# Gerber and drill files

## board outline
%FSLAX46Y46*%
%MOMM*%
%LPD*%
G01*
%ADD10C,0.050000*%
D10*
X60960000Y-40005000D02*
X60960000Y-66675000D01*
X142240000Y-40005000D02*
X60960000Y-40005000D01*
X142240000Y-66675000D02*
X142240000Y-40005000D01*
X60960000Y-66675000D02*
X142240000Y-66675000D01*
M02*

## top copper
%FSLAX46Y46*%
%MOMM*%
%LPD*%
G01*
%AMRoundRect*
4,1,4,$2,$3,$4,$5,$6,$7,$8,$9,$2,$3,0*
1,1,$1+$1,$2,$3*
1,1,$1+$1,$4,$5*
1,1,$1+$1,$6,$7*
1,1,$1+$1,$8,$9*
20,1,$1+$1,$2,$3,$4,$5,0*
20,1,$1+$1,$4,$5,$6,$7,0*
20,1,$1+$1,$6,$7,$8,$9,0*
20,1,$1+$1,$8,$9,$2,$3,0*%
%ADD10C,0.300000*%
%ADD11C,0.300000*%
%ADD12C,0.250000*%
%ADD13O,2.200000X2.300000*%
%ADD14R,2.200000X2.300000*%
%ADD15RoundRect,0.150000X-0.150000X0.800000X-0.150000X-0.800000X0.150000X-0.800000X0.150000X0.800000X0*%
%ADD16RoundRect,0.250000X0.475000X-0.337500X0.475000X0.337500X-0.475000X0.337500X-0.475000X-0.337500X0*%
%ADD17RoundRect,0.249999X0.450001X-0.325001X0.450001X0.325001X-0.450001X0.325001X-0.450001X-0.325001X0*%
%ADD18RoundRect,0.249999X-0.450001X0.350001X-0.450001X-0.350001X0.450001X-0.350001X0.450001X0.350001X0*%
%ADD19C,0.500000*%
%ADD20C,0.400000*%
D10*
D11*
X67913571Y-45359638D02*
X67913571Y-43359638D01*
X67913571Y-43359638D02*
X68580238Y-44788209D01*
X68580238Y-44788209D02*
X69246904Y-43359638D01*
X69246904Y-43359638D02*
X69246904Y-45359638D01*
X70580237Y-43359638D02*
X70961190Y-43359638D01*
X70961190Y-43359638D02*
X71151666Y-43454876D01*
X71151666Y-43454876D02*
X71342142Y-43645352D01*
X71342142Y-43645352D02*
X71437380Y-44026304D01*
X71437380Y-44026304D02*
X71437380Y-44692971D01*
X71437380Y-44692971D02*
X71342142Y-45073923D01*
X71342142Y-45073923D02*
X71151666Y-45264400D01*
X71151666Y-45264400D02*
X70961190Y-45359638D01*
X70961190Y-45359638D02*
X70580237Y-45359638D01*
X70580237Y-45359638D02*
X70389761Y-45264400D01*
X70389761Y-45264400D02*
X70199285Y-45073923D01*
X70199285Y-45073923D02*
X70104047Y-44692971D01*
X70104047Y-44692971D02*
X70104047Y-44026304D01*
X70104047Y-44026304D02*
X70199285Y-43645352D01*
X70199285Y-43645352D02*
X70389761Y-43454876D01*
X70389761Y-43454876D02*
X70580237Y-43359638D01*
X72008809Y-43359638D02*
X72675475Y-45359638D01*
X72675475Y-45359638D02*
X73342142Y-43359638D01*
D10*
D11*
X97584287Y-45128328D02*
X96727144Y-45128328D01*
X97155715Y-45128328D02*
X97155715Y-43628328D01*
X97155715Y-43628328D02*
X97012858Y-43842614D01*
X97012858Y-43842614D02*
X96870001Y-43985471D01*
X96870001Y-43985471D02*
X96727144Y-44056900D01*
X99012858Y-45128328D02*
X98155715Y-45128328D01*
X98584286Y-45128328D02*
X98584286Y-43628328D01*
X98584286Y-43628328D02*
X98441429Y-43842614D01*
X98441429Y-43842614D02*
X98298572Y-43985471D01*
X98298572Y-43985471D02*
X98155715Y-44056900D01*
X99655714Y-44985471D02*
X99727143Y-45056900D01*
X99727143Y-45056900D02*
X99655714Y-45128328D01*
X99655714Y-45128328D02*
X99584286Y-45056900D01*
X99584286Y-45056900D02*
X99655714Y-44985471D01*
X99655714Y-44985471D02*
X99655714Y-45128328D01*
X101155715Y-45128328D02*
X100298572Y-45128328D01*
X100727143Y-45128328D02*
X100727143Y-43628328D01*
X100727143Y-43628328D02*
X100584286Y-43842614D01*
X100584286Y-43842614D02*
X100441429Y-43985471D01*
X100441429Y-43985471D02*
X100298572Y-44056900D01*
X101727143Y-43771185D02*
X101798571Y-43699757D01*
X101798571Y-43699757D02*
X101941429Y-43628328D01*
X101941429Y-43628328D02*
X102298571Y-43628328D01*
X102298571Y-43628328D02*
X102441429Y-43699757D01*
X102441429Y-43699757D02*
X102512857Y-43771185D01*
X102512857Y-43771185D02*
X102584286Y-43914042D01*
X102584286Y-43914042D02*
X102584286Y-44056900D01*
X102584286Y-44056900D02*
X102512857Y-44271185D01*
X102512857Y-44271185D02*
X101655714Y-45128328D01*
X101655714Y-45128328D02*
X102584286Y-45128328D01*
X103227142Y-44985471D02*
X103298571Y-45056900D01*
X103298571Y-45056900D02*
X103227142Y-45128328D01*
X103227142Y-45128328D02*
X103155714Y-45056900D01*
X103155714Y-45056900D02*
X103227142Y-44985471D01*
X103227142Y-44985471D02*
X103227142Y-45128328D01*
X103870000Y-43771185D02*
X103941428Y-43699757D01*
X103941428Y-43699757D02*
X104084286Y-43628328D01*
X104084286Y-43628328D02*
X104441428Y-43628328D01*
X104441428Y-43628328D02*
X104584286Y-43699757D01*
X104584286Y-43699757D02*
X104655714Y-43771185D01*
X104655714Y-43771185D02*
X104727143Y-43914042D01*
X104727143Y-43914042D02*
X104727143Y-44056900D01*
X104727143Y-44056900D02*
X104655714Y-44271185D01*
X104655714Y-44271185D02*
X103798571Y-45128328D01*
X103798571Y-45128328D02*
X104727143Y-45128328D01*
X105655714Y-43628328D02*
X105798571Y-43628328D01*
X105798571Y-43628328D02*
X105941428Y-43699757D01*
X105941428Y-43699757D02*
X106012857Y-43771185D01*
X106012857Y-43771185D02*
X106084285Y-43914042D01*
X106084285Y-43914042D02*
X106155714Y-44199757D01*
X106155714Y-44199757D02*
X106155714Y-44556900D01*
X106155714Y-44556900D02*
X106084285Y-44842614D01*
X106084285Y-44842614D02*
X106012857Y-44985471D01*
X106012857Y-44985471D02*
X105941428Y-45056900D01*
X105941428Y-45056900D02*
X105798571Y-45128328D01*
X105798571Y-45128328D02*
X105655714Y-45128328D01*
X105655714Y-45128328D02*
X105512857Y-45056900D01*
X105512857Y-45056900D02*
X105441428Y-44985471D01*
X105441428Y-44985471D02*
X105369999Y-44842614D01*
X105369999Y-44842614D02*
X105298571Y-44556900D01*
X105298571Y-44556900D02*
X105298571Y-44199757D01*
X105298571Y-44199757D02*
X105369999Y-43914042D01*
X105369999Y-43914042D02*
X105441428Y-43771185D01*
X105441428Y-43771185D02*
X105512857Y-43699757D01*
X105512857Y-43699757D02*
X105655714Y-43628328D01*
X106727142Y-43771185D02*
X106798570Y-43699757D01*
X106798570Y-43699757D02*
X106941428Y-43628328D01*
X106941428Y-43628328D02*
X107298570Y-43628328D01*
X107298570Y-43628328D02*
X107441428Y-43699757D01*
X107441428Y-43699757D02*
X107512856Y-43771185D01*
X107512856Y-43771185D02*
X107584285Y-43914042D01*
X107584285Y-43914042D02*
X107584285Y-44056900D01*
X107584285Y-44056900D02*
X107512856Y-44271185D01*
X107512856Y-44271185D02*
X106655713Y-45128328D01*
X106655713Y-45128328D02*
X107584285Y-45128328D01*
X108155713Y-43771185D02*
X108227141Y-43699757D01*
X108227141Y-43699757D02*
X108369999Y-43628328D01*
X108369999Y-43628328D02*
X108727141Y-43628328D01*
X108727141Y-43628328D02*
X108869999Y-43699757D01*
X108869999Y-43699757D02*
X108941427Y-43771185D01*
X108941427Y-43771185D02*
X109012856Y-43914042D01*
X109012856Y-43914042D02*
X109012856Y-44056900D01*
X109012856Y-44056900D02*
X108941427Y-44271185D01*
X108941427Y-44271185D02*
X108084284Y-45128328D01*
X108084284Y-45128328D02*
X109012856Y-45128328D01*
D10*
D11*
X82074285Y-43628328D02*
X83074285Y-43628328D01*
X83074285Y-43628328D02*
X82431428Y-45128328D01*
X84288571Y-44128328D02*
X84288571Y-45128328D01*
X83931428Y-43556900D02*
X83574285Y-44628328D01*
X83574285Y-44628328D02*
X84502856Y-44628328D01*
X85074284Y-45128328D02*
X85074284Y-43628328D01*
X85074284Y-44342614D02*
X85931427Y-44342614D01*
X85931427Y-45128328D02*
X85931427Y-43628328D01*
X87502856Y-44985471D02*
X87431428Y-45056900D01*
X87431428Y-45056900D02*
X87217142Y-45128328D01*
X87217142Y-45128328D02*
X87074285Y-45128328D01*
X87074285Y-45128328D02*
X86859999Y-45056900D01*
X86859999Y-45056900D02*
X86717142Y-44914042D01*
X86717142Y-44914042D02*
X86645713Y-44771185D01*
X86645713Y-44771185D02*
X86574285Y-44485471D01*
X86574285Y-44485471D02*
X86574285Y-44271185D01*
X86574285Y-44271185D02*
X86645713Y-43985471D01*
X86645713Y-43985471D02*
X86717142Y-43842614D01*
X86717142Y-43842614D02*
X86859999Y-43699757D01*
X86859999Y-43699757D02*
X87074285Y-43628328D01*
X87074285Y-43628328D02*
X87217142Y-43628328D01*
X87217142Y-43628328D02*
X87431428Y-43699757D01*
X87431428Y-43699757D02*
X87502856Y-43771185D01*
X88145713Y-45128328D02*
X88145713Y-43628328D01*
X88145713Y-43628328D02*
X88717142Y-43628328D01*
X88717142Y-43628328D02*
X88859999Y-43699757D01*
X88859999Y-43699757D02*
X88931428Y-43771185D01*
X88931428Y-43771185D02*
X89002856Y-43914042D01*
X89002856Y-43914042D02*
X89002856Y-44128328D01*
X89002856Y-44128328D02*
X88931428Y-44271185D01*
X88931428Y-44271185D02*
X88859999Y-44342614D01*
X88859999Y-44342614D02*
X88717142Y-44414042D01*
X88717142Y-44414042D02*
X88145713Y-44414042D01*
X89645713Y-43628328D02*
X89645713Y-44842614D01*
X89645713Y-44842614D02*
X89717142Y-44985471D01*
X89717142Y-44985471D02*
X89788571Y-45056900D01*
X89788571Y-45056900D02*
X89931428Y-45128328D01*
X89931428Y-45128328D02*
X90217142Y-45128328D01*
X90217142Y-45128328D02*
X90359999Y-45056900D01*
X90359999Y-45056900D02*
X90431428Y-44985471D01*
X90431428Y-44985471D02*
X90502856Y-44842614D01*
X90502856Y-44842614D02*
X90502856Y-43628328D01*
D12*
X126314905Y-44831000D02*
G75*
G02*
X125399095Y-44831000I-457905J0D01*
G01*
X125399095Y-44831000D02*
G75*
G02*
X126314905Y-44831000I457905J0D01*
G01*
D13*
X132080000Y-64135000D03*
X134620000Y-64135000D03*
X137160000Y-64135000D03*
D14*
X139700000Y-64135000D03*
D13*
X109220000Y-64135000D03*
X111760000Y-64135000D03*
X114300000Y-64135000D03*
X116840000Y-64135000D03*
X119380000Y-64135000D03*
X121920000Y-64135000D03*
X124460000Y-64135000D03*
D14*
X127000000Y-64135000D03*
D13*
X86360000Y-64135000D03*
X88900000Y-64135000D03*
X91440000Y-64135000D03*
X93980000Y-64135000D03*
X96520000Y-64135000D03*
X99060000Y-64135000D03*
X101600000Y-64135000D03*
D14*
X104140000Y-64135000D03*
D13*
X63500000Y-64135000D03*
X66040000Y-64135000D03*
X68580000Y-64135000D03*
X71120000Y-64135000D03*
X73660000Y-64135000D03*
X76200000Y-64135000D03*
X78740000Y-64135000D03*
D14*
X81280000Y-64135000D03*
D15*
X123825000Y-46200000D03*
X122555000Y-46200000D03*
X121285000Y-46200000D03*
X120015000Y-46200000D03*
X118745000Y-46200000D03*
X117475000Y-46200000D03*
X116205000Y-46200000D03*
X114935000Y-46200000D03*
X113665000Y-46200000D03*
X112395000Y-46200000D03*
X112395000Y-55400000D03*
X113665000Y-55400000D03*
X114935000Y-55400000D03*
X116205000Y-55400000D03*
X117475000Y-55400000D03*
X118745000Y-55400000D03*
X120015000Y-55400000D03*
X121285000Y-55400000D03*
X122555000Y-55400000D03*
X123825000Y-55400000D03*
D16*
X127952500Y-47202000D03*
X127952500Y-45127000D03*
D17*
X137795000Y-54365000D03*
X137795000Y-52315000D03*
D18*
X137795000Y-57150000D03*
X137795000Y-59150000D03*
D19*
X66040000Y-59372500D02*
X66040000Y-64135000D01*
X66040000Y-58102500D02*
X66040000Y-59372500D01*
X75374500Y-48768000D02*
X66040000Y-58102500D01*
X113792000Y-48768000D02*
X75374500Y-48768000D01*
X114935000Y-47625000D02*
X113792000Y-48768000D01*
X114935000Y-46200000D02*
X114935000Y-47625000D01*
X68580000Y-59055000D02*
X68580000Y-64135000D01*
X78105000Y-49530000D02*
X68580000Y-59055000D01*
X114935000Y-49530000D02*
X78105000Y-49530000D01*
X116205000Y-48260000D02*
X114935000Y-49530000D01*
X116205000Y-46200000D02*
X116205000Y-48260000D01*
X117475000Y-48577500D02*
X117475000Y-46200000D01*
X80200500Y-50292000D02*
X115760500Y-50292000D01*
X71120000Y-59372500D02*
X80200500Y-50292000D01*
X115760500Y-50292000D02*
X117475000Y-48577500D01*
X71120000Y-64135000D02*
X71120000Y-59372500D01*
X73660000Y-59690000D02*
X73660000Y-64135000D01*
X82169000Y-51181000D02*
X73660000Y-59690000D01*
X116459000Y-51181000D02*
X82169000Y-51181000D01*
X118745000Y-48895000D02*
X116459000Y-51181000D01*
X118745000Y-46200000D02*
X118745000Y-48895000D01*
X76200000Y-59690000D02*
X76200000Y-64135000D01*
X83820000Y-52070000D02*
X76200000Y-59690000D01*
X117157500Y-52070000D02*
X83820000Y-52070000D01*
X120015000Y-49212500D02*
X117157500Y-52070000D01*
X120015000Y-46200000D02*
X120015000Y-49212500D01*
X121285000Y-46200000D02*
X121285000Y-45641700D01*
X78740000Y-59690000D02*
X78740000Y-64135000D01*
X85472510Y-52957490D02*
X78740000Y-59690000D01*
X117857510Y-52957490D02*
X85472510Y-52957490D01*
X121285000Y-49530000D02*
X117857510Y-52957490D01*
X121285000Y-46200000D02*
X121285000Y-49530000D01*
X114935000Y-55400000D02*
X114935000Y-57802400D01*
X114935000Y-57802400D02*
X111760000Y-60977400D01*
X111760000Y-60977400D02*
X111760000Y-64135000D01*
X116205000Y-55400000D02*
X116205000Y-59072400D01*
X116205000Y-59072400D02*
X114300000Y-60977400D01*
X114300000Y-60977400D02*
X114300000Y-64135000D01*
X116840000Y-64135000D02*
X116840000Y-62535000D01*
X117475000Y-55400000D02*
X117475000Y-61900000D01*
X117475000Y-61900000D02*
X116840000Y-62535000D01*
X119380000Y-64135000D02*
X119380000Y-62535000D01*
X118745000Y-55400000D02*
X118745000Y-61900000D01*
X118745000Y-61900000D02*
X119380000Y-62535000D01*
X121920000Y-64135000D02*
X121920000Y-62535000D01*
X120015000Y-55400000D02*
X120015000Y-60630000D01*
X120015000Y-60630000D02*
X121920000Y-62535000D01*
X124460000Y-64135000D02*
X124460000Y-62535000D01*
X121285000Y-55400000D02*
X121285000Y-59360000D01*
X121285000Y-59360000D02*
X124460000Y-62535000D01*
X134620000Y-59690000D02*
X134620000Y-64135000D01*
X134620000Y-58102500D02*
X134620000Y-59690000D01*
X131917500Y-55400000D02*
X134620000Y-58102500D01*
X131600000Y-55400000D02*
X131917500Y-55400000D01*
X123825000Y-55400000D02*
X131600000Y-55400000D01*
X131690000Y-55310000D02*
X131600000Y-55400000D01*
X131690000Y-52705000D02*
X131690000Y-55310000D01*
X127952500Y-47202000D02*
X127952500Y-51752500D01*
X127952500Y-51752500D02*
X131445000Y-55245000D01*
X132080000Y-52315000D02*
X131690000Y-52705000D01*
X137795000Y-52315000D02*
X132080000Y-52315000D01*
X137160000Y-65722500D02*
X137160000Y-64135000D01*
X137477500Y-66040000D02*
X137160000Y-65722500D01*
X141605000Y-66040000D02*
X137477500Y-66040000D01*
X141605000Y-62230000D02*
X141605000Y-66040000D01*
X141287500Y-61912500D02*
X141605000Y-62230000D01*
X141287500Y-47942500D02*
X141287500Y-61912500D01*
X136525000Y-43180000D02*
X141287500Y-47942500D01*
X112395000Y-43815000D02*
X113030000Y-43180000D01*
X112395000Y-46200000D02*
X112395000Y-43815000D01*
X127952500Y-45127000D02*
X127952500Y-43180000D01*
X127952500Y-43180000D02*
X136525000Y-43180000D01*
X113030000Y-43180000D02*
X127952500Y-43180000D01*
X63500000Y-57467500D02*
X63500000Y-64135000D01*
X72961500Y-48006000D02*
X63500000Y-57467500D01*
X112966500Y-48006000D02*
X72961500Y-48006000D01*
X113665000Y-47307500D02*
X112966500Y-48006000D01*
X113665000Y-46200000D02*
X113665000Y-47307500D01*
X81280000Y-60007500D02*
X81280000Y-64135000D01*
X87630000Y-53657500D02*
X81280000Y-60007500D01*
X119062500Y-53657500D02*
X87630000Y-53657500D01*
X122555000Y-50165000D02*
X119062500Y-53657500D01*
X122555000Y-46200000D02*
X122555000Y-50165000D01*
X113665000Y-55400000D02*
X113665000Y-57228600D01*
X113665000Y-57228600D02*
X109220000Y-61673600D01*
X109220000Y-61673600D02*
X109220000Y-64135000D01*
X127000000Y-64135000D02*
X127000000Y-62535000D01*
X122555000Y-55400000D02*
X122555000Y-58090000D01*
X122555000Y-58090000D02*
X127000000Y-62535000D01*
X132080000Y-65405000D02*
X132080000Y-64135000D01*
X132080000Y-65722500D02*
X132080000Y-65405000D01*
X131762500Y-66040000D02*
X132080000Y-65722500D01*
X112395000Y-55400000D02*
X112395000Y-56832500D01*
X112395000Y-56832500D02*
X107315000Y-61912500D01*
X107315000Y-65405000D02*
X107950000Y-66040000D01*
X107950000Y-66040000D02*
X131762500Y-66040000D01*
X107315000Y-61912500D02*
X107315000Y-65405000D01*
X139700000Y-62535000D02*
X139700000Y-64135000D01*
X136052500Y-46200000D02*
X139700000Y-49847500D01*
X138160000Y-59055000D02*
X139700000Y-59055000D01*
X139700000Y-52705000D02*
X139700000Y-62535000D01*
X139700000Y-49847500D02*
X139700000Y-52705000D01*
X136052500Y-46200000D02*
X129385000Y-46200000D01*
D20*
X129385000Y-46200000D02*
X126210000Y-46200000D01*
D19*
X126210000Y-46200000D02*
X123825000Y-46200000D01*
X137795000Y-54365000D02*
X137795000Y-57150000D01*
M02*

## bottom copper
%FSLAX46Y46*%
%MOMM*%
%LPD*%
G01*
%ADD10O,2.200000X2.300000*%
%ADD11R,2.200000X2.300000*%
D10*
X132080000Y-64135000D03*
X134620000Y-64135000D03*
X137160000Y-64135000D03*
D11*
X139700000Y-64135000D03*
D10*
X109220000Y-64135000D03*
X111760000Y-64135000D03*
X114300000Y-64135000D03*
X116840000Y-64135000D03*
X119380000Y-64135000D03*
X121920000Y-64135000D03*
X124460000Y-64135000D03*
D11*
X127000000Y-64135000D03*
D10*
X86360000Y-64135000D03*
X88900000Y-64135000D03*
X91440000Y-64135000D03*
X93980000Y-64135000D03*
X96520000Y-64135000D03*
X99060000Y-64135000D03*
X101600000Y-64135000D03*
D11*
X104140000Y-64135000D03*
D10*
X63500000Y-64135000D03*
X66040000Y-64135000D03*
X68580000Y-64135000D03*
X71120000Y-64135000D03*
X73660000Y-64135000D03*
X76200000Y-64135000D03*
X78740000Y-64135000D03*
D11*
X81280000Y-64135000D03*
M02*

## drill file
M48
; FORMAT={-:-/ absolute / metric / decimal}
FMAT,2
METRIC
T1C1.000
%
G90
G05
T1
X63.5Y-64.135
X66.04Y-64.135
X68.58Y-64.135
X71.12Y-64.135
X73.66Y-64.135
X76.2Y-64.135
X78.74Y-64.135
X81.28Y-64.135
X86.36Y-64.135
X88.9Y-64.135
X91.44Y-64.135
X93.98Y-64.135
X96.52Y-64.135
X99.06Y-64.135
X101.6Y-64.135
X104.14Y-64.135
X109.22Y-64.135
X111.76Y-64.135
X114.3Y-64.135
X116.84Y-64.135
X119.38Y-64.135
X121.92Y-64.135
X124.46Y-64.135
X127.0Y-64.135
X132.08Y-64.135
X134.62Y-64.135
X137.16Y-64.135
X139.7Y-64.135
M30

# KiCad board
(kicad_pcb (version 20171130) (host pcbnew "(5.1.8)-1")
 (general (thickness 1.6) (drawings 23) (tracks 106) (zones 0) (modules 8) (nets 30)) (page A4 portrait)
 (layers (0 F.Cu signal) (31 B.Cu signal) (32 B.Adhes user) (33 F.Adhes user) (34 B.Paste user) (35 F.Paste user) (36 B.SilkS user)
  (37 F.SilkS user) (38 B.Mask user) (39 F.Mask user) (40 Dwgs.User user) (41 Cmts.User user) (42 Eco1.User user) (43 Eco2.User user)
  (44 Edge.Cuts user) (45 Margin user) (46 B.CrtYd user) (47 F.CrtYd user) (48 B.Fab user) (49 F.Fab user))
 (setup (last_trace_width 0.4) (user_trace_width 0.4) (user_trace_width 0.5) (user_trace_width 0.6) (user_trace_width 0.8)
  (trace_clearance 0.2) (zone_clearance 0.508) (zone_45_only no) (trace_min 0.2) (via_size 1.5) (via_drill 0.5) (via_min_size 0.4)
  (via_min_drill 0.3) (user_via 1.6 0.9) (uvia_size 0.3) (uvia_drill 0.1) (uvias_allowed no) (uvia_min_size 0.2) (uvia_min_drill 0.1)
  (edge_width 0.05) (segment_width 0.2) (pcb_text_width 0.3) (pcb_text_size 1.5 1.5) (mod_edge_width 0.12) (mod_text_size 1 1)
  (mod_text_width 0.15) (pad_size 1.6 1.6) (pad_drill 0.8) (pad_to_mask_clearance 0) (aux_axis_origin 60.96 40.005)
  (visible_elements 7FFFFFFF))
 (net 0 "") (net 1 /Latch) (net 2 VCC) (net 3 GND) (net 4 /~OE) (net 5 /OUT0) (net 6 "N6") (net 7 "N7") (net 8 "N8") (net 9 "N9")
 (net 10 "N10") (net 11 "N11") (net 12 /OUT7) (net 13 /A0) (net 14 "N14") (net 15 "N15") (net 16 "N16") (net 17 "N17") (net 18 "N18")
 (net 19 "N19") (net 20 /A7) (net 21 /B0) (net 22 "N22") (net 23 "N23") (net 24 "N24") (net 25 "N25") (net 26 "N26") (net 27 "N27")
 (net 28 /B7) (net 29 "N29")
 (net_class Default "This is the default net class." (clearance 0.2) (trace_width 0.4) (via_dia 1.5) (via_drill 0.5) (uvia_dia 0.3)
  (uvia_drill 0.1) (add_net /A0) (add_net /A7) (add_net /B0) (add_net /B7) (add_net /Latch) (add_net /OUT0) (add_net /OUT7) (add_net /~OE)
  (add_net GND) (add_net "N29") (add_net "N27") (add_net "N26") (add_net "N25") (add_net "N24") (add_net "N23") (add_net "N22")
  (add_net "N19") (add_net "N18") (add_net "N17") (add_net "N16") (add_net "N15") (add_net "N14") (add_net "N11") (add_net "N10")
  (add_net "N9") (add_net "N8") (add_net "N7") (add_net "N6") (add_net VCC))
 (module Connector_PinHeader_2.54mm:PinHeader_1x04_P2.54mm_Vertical (layer F.Cu) (at 139.7 64.135 270)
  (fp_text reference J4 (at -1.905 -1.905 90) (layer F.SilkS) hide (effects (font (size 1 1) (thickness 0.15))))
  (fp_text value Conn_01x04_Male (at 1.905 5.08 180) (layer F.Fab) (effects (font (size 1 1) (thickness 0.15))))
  (pad 4 thru_hole oval (at 0 7.62 270) (size 2.3 2.2) (drill 1) (layers *.Cu *.Mask) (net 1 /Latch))
  (pad 3 thru_hole oval (at 0 5.08 270) (size 2.3 2.2) (drill 1) (layers *.Cu *.Mask) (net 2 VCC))
  (pad 2 thru_hole oval (at 0 2.54 270) (size 2.3 2.2) (drill 1) (layers *.Cu *.Mask) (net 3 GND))
  (pad 1 thru_hole rect (at 0 0 270) (size 2.3 2.2) (drill 1) (layers *.Cu *.Mask) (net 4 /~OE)))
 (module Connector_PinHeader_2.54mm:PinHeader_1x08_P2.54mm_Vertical (layer F.Cu) (at 127 64.135 270)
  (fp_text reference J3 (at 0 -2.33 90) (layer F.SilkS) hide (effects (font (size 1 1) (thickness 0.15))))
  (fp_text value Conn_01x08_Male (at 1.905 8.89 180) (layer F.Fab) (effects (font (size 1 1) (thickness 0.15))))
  (pad 8 thru_hole oval (at 0 17.78 270) (size 2.3 2.2) (drill 1) (layers *.Cu *.Mask) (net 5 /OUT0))
  (pad 7 thru_hole oval (at 0 15.24 270) (size 2.3 2.2) (drill 1) (layers *.Cu *.Mask) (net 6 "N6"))
  (pad 6 thru_hole oval (at 0 12.7 270) (size 2.3 2.2) (drill 1) (layers *.Cu *.Mask) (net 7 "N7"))
  (pad 5 thru_hole oval (at 0 10.16 270) (size 2.3 2.2) (drill 1) (layers *.Cu *.Mask) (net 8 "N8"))
  (pad 4 thru_hole oval (at 0 7.62 270) (size 2.3 2.2) (drill 1) (layers *.Cu *.Mask) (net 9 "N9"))
  (pad 3 thru_hole oval (at 0 5.08 270) (size 2.3 2.2) (drill 1) (layers *.Cu *.Mask) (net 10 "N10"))
  (pad 2 thru_hole oval (at 0 2.54 270) (size 2.3 2.2) (drill 1) (layers *.Cu *.Mask) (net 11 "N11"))
  (pad 1 thru_hole rect (at 0 0 270) (size 2.3 2.2) (drill 1) (layers *.Cu *.Mask) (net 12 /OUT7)))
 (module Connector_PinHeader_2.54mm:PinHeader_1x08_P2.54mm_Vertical (layer F.Cu) (at 104.14 64.135 270)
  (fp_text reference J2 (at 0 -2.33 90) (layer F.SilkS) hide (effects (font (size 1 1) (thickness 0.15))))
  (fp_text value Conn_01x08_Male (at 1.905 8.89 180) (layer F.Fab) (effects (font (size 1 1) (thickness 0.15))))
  (pad 8 thru_hole oval (at 0 17.78 270) (size 2.3 2.2) (drill 1) (layers *.Cu *.Mask) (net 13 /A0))
  (pad 7 thru_hole oval (at 0 15.24 270) (size 2.3 2.2) (drill 1) (layers *.Cu *.Mask) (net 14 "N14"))
  (pad 6 thru_hole oval (at 0 12.7 270) (size 2.3 2.2) (drill 1) (layers *.Cu *.Mask) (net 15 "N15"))
  (pad 5 thru_hole oval (at 0 10.16 270) (size 2.3 2.2) (drill 1) (layers *.Cu *.Mask) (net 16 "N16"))
  (pad 4 thru_hole oval (at 0 7.62 270) (size 2.3 2.2) (drill 1) (layers *.Cu *.Mask) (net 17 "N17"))
  (pad 3 thru_hole oval (at 0 5.08 270) (size 2.3 2.2) (drill 1) (layers *.Cu *.Mask) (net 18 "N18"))
  (pad 2 thru_hole oval (at 0 2.54 270) (size 2.3 2.2) (drill 1) (layers *.Cu *.Mask) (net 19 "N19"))
  (pad 1 thru_hole rect (at 0 0 270) (size 2.3 2.2) (drill 1) (layers *.Cu *.Mask) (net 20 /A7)))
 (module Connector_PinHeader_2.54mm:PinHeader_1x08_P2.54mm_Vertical (layer F.Cu) (at 81.28 64.135 270)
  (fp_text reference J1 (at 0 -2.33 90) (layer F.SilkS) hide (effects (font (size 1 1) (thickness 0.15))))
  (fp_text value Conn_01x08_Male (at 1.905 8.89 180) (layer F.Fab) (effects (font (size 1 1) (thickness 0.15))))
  (pad 8 thru_hole oval (at 0 17.78 270) (size 2.3 2.2) (drill 1) (layers *.Cu *.Mask) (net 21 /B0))
  (pad 7 thru_hole oval (at 0 15.24 270) (size 2.3 2.2) (drill 1) (layers *.Cu *.Mask) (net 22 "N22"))
  (pad 6 thru_hole oval (at 0 12.7 270) (size 2.3 2.2) (drill 1) (layers *.Cu *.Mask) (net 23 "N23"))
  (pad 5 thru_hole oval (at 0 10.16 270) (size 2.3 2.2) (drill 1) (layers *.Cu *.Mask) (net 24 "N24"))
  (pad 4 thru_hole oval (at 0 7.62 270) (size 2.3 2.2) (drill 1) (layers *.Cu *.Mask) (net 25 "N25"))
  (pad 3 thru_hole oval (at 0 5.08 270) (size 2.3 2.2) (drill 1) (layers *.Cu *.Mask) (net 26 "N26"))
  (pad 2 thru_hole oval (at 0 2.54 270) (size 2.3 2.2) (drill 1) (layers *.Cu *.Mask) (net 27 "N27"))
  (pad 1 thru_hole rect (at 0 0 270) (size 2.3 2.2) (drill 1) (layers *.Cu *.Mask) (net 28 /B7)))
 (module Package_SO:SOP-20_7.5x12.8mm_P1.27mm (layer F.Cu) (at 118.11 50.8 270)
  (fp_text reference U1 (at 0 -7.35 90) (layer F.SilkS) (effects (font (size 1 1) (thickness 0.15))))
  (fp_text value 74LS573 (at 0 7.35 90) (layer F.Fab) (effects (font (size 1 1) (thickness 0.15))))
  (pad 1 smd roundrect (at -4.6 -5.715 270) (size 1.9 0.6) (layers F.Cu F.Paste F.Mask) (roundrect_rratio 0.25) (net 4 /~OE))
  (pad 2 smd roundrect (at -4.6 -4.445 270) (size 1.9 0.6) (layers F.Cu F.Paste F.Mask) (roundrect_rratio 0.25) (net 28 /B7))
  (pad 3 smd roundrect (at -4.6 -3.175 270) (size 1.9 0.6) (layers F.Cu F.Paste F.Mask) (roundrect_rratio 0.25) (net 27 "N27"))
  (pad 4 smd roundrect (at -4.6 -1.905 270) (size 1.9 0.6) (layers F.Cu F.Paste F.Mask) (roundrect_rratio 0.25) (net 26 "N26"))
  (pad 5 smd roundrect (at -4.6 -0.635 270) (size 1.9 0.6) (layers F.Cu F.Paste F.Mask) (roundrect_rratio 0.25) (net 25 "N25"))
  (pad 6 smd roundrect (at -4.6 0.635 270) (size 1.9 0.6) (layers F.Cu F.Paste F.Mask) (roundrect_rratio 0.25) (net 24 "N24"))
  (pad 7 smd roundrect (at -4.6 1.905 270) (size 1.9 0.6) (layers F.Cu F.Paste F.Mask) (roundrect_rratio 0.25) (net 23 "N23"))
  (pad 8 smd roundrect (at -4.6 3.175 270) (size 1.9 0.6) (layers F.Cu F.Paste F.Mask) (roundrect_rratio 0.25) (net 22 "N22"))
  (pad 9 smd roundrect (at -4.6 4.445 270) (size 1.9 0.6) (layers F.Cu F.Paste F.Mask) (roundrect_rratio 0.25) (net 21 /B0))
  (pad 10 smd roundrect (at -4.6 5.715 270) (size 1.9 0.6) (layers F.Cu F.Paste F.Mask) (roundrect_rratio 0.25) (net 3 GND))
  (pad 11 smd roundrect (at 4.6 5.715 270) (size 1.9 0.6) (layers F.Cu F.Paste F.Mask) (roundrect_rratio 0.25) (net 1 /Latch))
  (pad 12 smd roundrect (at 4.6 4.445 270) (size 1.9 0.6) (layers F.Cu F.Paste F.Mask) (roundrect_rratio 0.25) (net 5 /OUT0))
  (pad 13 smd roundrect (at 4.6 3.175 270) (size 1.9 0.6) (layers F.Cu F.Paste F.Mask) (roundrect_rratio 0.25) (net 6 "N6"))
  (pad 14 smd roundrect (at 4.6 1.905 270) (size 1.9 0.6) (layers F.Cu F.Paste F.Mask) (roundrect_rratio 0.25) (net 7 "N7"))
  (pad 15 smd roundrect (at 4.6 0.635 270) (size 1.9 0.6) (layers F.Cu F.Paste F.Mask) (roundrect_rratio 0.25) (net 8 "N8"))
  (pad 16 smd roundrect (at 4.6 -0.635 270) (size 1.9 0.6) (layers F.Cu F.Paste F.Mask) (roundrect_rratio 0.25) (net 9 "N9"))
  (pad 17 smd roundrect (at 4.6 -1.905 270) (size 1.9 0.6) (layers F.Cu F.Paste F.Mask) (roundrect_rratio 0.25) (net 10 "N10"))
  (pad 18 smd roundrect (at 4.6 -3.175 270) (size 1.9 0.6) (layers F.Cu F.Paste F.Mask) (roundrect_rratio 0.25) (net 11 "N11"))
  (pad 19 smd roundrect (at 4.6 -4.445 270) (size 1.9 0.6) (layers F.Cu F.Paste F.Mask) (roundrect_rratio 0.25) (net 12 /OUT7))
  (pad 20 smd roundrect (at 4.6 -5.715 270) (size 1.9 0.6) (layers F.Cu F.Paste F.Mask) (roundrect_rratio 0.25) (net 2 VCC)))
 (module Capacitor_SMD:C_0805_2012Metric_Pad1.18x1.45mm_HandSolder (layer F.Cu) (at 127.9525 46.1645 90)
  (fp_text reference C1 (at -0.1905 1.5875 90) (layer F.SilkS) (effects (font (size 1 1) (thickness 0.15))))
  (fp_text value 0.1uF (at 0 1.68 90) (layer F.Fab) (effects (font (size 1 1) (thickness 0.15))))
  (pad 1 smd roundrect (at -1.0375 0 90) (size 1.175 1.45) (layers F.Cu F.Paste F.Mask) (roundrect_rratio 0.2127659574468085) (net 2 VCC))
  (pad 2 smd roundrect (at 1.0375 0 90) (size 1.175 1.45) (layers F.Cu F.Paste F.Mask) (roundrect_rratio 0.2127659574468085) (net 3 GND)))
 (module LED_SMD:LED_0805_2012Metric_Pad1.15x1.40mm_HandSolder (layer F.Cu) (at 137.795 53.34 90)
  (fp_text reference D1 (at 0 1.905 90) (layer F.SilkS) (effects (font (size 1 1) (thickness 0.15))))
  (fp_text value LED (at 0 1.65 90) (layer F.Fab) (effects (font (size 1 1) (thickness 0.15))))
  (pad 1 smd roundrect (at -1.025 0 90) (size 1.15 1.4) (layers F.Cu F.Paste F.Mask) (roundrect_rratio 0.2173904347826087) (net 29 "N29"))
  (pad 2 smd roundrect (at 1.025 0 90) (size 1.15 1.4) (layers F.Cu F.Paste F.Mask) (roundrect_rratio 0.2173904347826087) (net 2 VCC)))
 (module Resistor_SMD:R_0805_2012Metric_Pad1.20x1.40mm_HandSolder (layer F.Cu) (at 137.795 58.15 270)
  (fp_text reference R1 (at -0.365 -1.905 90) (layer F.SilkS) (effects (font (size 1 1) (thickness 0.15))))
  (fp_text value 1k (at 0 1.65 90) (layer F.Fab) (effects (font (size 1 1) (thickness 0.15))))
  (pad 1 smd roundrect (at -1 0 270) (size 1.2 1.4) (layers F.Cu F.Paste F.Mask) (roundrect_rratio 0.2083325) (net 29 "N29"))
  (pad 2 smd roundrect (at 1 0 270) (size 1.2 1.4) (layers F.Cu F.Paste F.Mask) (roundrect_rratio 0.2083325) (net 4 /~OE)))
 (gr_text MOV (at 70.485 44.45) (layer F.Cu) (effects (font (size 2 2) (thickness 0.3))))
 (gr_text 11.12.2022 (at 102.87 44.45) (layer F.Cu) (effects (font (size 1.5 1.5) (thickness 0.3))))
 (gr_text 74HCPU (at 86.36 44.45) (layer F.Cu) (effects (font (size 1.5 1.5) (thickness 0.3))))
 (gr_circle (center 125.857 44.831) (end 126.314905 44.831) (layer F.Cu) (width 0.25))
 (gr_line (start 60.96 40.005) (end 60.96 66.675) (layer Edge.Cuts) (width 0.05))
 (gr_line (start 142.24 40.005) (end 60.96 40.005) (layer Edge.Cuts) (width 0.05))
 (gr_line (start 142.24 66.675) (end 142.24 40.005) (layer Edge.Cuts) (width 0.05))
 (gr_line (start 60.96 66.675) (end 142.24 66.675) (layer Edge.Cuts) (width 0.05))
 (segment (start 66.04 59.3725) (end 66.04 64.135) (width 0.5) (layer F.Cu) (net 22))
 (segment (start 66.04 58.1025) (end 66.04 59.3725) (width 0.5) (layer F.Cu) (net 22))
 (segment (start 75.3745 48.768) (end 66.04 58.1025) (width 0.5) (layer F.Cu) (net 22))
 (segment (start 113.792 48.768) (end 75.3745 48.768) (width 0.5) (layer F.Cu) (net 22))
 (segment (start 114.935 47.625) (end 113.792 48.768) (width 0.5) (layer F.Cu) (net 22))
 (segment (start 114.935 46.2) (end 114.935 47.625) (width 0.5) (layer F.Cu) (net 22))
 (segment (start 68.58 59.055) (end 68.58 64.135) (width 0.5) (layer F.Cu) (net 23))
 (segment (start 78.105 49.53) (end 68.58 59.055) (width 0.5) (layer F.Cu) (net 23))
 (segment (start 114.935 49.53) (end 78.105 49.53) (width 0.5) (layer F.Cu) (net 23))
 (segment (start 116.205 48.26) (end 114.935 49.53) (width 0.5) (layer F.Cu) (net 23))
 (segment (start 116.205 46.2) (end 116.205 48.26) (width 0.5) (layer F.Cu) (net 23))
 (segment (start 117.475 48.5775) (end 117.475 46.2) (width 0.5) (layer F.Cu) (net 24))
 (segment (start 80.2005 50.292) (end 115.7605 50.292) (width 0.5) (layer F.Cu) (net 24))
 (segment (start 71.12 59.3725) (end 80.2005 50.292) (width 0.5) (layer F.Cu) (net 24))
 (segment (start 115.7605 50.292) (end 117.475 48.5775) (width 0.5) (layer F.Cu) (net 24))
 (segment (start 71.12 64.135) (end 71.12 59.3725) (width 0.5) (layer F.Cu) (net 24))
 (segment (start 73.66 59.69) (end 73.66 64.135) (width 0.5) (layer F.Cu) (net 25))
 (segment (start 82.169 51.181) (end 73.66 59.69) (width 0.5) (layer F.Cu) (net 25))
 (segment (start 116.459 51.181) (end 82.169 51.181) (width 0.5) (layer F.Cu) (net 25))
 (segment (start 118.745 48.895) (end 116.459 51.181) (width 0.5) (layer F.Cu) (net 25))
 (segment (start 118.745 46.2) (end 118.745 48.895) (width 0.5) (layer F.Cu) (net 25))
 (segment (start 76.2 59.69) (end 76.2 64.135) (width 0.5) (layer F.Cu) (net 26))
 (segment (start 83.82 52.07) (end 76.2 59.69) (width 0.5) (layer F.Cu) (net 26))
 (segment (start 117.1575 52.07) (end 83.82 52.07) (width 0.5) (layer F.Cu) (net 26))
 (segment (start 120.015 49.2125) (end 117.1575 52.07) (width 0.5) (layer F.Cu) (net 26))
 (segment (start 120.015 46.2) (end 120.015 49.2125) (width 0.5) (layer F.Cu) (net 26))
 (segment (start 121.285 46.2) (end 121.285 45.6417) (width 0.5) (layer F.Cu) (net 27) (status 30))
 (segment (start 78.74 59.69) (end 78.74 64.135) (width 0.5) (layer F.Cu) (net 27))
 (segment (start 85.47251 52.95749) (end 78.74 59.69) (width 0.5) (layer F.Cu) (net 27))
 (segment (start 117.85751 52.95749) (end 85.47251 52.95749) (width 0.5) (layer F.Cu) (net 27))
 (segment (start 121.285 49.53) (end 117.85751 52.95749) (width 0.5) (layer F.Cu) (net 27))
 (segment (start 121.285 46.2) (end 121.285 49.53) (width 0.5) (layer F.Cu) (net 27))
 (segment (start 114.935 55.4) (end 114.935 57.8024) (width 0.5) (layer F.Cu) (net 6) (status 10))
 (segment (start 114.935 57.8024) (end 111.76 60.9774) (width 0.5) (layer F.Cu) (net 6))
 (segment (start 111.76 60.9774) (end 111.76 64.135) (width 0.5) (layer F.Cu) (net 6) (status 20))
 (segment (start 116.205 55.4) (end 116.205 59.0724) (width 0.5) (layer F.Cu) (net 7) (status 10))
 (segment (start 116.205 59.0724) (end 114.3 60.9774) (width 0.5) (layer F.Cu) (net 7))
 (segment (start 114.3 60.9774) (end 114.3 64.135) (width 0.5) (layer F.Cu) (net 7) (status 20))
 (segment (start 116.84 64.135) (end 116.84 62.535) (width 0.5) (layer F.Cu) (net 8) (status 10))
 (segment (start 117.475 55.4) (end 117.475 61.9) (width 0.5) (layer F.Cu) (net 8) (status 10))
 (segment (start 117.475 61.9) (end 116.84 62.535) (width 0.5) (layer F.Cu) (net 8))
 (segment (start 119.38 64.135) (end 119.38 62.535) (width 0.5) (layer F.Cu) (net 9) (status 10))
 (segment (start 118.745 55.4) (end 118.745 61.9) (width 0.5) (layer F.Cu) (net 9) (status 10))
 (segment (start 118.745 61.9) (end 119.38 62.535) (width 0.5) (layer F.Cu) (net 9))
 (segment (start 121.92 64.135) (end 121.92 62.535) (width 0.5) (layer F.Cu) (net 10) (status 10))
 (segment (start 120.015 55.4) (end 120.015 60.63) (width 0.5) (layer F.Cu) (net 10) (status 10))
 (segment (start 120.015 60.63) (end 121.92 62.535) (width 0.5) (layer F.Cu) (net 10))
 (segment (start 124.46 64.135) (end 124.46 62.535) (width 0.5) (layer F.Cu) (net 11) (status 10))
 (segment (start 121.285 55.4) (end 121.285 59.36) (width 0.5) (layer F.Cu) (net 11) (status 10))
 (segment (start 121.285 59.36) (end 124.46 62.535) (width 0.5) (layer F.Cu) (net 11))
 (segment (start 134.62 59.69) (end 134.62 64.135) (width 0.5) (layer F.Cu) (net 2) (status 20))
 (segment (start 134.62 58.1025) (end 134.62 59.69) (width 0.5) (layer F.Cu) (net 2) (status 10))
 (segment (start 131.9175 55.4) (end 134.62 58.1025) (width 0.5) (layer F.Cu) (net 2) (status 20))
 (segment (start 131.6 55.4) (end 131.9175 55.4) (width 0.5) (layer F.Cu) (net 2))
 (segment (start 123.825 55.4) (end 131.6 55.4) (width 0.5) (layer F.Cu) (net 2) (status 10))
 (segment (start 131.69 55.31) (end 131.6 55.4) (width 0.5) (layer F.Cu) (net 2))
 (segment (start 131.69 52.705) (end 131.69 55.31) (width 0.5) (layer F.Cu) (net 2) (status 10))
 (segment (start 127.9525 47.202) (end 127.9525 51.7525) (width 0.5) (layer F.Cu) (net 2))
 (segment (start 127.9525 51.7525) (end 131.445 55.245) (width 0.5) (layer F.Cu) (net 2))
 (segment (start 132.08 52.315) (end 131.69 52.705) (width 0.5) (layer F.Cu) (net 2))
 (segment (start 137.795 52.315) (end 132.08 52.315) (width 0.5) (layer F.Cu) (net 2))
 (segment (start 137.16 65.7225) (end 137.16 64.135) (width 0.5) (layer F.Cu) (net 3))
 (segment (start 137.4775 66.04) (end 137.16 65.7225) (width 0.5) (layer F.Cu) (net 3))
 (segment (start 141.605 66.04) (end 137.4775 66.04) (width 0.5) (layer F.Cu) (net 3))
 (segment (start 141.605 62.23) (end 141.605 66.04) (width 0.5) (layer F.Cu) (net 3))
 (segment (start 141.2875 61.9125) (end 141.605 62.23) (width 0.5) (layer F.Cu) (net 3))
 (segment (start 141.2875 47.9425) (end 141.2875 61.9125) (width 0.5) (layer F.Cu) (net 3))
 (segment (start 136.525 43.18) (end 141.2875 47.9425) (width 0.5) (layer F.Cu) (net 3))
 (segment (start 112.395 43.815) (end 113.03 43.18) (width 0.5) (layer F.Cu) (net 3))
 (segment (start 112.395 46.2) (end 112.395 43.815) (width 0.5) (layer F.Cu) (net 3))
 (segment (start 127.9525 45.127) (end 127.9525 43.18) (width 0.5) (layer F.Cu) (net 3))
 (segment (start 127.9525 43.18) (end 136.525 43.18) (width 0.5) (layer F.Cu) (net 3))
 (segment (start 113.03 43.18) (end 127.9525 43.18) (width 0.5) (layer F.Cu) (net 3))
 (segment (start 63.5 57.4675) (end 63.5 64.135) (width 0.5) (layer F.Cu) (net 21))
 (segment (start 72.9615 48.006) (end 63.5 57.4675) (width 0.5) (layer F.Cu) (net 21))
 (segment (start 112.9665 48.006) (end 72.9615 48.006) (width 0.5) (layer F.Cu) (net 21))
 (segment (start 113.665 47.3075) (end 112.9665 48.006) (width 0.5) (layer F.Cu) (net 21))
 (segment (start 113.665 46.2) (end 113.665 47.3075) (width 0.5) (layer F.Cu) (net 21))
 (segment (start 81.28 60.0075) (end 81.28 64.135) (width 0.5) (layer F.Cu) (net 28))
 (segment (start 87.63 53.6575) (end 81.28 60.0075) (width 0.5) (layer F.Cu) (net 28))
 (segment (start 119.0625 53.6575) (end 87.63 53.6575) (width 0.5) (layer F.Cu) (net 28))
 (segment (start 122.555 50.165) (end 119.0625 53.6575) (width 0.5) (layer F.Cu) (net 28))
 (segment (start 122.555 46.2) (end 122.555 50.165) (width 0.5) (layer F.Cu) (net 28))
 (segment (start 113.665 55.4) (end 113.665 57.2286) (width 0.5) (layer F.Cu) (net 5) (status 10))
 (segment (start 113.665 57.2286) (end 109.22 61.6736) (width 0.5) (layer F.Cu) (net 5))
 (segment (start 109.22 61.6736) (end 109.22 64.135) (width 0.5) (layer F.Cu) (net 5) (status 20))
 (segment (start 127 64.135) (end 127 62.535) (width 0.5) (layer F.Cu) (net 12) (status 10))
 (segment (start 122.555 55.4) (end 122.555 58.09) (width 0.5) (layer F.Cu) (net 12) (status 10))
 (segment (start 122.555 58.09) (end 127 62.535) (width 0.5) (layer F.Cu) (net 12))
 (segment (start 132.08 65.405) (end 132.08 64.135) (width 0.5) (layer F.Cu) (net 1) (status 20))
 (segment (start 132.08 65.7225) (end 132.08 65.405) (width 0.5) (layer F.Cu) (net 1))
 (segment (start 131.7625 66.04) (end 132.08 65.7225) (width 0.5) (layer F.Cu) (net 1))
 (segment (start 112.395 55.4) (end 112.395 56.8325) (width 0.5) (layer F.Cu) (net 1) (status 10))
 (segment (start 112.395 56.8325) (end 107.315 61.9125) (width 0.5) (layer F.Cu) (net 1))
 (segment (start 107.315 65.405) (end 107.95 66.04) (width 0.5) (layer F.Cu) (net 1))
 (segment (start 107.95 66.04) (end 131.7625 66.04) (width 0.5) (layer F.Cu) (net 1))
 (segment (start 107.315 61.9125) (end 107.315 65.405) (width 0.5) (layer F.Cu) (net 1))
 (segment (start 139.7 62.535) (end 139.7 64.135) (width 0.5) (layer F.Cu) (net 4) (status 20))
 (segment (start 136.0525 46.2) (end 139.7 49.8475) (width 0.5) (layer F.Cu) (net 4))
 (segment (start 138.16 59.055) (end 139.7 59.055) (width 0.5) (layer F.Cu) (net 4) (status 10))
 (segment (start 139.7 52.705) (end 139.7 62.535) (width 0.5) (layer F.Cu) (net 4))
 (segment (start 139.7 49.8475) (end 139.7 52.705) (width 0.5) (layer F.Cu) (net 4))
 (segment (start 136.0525 46.2) (end 129.385 46.2) (width 0.5) (layer F.Cu) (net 4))
 (segment (start 129.385 46.2) (end 126.21 46.2) (width 0.4) (layer F.Cu) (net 4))
 (segment (start 126.21 46.2) (end 123.825 46.2) (width 0.5) (layer F.Cu) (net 4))
 (segment (start 137.795 54.365) (end 137.795 57.15) (width 0.5) (layer F.Cu) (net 29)))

